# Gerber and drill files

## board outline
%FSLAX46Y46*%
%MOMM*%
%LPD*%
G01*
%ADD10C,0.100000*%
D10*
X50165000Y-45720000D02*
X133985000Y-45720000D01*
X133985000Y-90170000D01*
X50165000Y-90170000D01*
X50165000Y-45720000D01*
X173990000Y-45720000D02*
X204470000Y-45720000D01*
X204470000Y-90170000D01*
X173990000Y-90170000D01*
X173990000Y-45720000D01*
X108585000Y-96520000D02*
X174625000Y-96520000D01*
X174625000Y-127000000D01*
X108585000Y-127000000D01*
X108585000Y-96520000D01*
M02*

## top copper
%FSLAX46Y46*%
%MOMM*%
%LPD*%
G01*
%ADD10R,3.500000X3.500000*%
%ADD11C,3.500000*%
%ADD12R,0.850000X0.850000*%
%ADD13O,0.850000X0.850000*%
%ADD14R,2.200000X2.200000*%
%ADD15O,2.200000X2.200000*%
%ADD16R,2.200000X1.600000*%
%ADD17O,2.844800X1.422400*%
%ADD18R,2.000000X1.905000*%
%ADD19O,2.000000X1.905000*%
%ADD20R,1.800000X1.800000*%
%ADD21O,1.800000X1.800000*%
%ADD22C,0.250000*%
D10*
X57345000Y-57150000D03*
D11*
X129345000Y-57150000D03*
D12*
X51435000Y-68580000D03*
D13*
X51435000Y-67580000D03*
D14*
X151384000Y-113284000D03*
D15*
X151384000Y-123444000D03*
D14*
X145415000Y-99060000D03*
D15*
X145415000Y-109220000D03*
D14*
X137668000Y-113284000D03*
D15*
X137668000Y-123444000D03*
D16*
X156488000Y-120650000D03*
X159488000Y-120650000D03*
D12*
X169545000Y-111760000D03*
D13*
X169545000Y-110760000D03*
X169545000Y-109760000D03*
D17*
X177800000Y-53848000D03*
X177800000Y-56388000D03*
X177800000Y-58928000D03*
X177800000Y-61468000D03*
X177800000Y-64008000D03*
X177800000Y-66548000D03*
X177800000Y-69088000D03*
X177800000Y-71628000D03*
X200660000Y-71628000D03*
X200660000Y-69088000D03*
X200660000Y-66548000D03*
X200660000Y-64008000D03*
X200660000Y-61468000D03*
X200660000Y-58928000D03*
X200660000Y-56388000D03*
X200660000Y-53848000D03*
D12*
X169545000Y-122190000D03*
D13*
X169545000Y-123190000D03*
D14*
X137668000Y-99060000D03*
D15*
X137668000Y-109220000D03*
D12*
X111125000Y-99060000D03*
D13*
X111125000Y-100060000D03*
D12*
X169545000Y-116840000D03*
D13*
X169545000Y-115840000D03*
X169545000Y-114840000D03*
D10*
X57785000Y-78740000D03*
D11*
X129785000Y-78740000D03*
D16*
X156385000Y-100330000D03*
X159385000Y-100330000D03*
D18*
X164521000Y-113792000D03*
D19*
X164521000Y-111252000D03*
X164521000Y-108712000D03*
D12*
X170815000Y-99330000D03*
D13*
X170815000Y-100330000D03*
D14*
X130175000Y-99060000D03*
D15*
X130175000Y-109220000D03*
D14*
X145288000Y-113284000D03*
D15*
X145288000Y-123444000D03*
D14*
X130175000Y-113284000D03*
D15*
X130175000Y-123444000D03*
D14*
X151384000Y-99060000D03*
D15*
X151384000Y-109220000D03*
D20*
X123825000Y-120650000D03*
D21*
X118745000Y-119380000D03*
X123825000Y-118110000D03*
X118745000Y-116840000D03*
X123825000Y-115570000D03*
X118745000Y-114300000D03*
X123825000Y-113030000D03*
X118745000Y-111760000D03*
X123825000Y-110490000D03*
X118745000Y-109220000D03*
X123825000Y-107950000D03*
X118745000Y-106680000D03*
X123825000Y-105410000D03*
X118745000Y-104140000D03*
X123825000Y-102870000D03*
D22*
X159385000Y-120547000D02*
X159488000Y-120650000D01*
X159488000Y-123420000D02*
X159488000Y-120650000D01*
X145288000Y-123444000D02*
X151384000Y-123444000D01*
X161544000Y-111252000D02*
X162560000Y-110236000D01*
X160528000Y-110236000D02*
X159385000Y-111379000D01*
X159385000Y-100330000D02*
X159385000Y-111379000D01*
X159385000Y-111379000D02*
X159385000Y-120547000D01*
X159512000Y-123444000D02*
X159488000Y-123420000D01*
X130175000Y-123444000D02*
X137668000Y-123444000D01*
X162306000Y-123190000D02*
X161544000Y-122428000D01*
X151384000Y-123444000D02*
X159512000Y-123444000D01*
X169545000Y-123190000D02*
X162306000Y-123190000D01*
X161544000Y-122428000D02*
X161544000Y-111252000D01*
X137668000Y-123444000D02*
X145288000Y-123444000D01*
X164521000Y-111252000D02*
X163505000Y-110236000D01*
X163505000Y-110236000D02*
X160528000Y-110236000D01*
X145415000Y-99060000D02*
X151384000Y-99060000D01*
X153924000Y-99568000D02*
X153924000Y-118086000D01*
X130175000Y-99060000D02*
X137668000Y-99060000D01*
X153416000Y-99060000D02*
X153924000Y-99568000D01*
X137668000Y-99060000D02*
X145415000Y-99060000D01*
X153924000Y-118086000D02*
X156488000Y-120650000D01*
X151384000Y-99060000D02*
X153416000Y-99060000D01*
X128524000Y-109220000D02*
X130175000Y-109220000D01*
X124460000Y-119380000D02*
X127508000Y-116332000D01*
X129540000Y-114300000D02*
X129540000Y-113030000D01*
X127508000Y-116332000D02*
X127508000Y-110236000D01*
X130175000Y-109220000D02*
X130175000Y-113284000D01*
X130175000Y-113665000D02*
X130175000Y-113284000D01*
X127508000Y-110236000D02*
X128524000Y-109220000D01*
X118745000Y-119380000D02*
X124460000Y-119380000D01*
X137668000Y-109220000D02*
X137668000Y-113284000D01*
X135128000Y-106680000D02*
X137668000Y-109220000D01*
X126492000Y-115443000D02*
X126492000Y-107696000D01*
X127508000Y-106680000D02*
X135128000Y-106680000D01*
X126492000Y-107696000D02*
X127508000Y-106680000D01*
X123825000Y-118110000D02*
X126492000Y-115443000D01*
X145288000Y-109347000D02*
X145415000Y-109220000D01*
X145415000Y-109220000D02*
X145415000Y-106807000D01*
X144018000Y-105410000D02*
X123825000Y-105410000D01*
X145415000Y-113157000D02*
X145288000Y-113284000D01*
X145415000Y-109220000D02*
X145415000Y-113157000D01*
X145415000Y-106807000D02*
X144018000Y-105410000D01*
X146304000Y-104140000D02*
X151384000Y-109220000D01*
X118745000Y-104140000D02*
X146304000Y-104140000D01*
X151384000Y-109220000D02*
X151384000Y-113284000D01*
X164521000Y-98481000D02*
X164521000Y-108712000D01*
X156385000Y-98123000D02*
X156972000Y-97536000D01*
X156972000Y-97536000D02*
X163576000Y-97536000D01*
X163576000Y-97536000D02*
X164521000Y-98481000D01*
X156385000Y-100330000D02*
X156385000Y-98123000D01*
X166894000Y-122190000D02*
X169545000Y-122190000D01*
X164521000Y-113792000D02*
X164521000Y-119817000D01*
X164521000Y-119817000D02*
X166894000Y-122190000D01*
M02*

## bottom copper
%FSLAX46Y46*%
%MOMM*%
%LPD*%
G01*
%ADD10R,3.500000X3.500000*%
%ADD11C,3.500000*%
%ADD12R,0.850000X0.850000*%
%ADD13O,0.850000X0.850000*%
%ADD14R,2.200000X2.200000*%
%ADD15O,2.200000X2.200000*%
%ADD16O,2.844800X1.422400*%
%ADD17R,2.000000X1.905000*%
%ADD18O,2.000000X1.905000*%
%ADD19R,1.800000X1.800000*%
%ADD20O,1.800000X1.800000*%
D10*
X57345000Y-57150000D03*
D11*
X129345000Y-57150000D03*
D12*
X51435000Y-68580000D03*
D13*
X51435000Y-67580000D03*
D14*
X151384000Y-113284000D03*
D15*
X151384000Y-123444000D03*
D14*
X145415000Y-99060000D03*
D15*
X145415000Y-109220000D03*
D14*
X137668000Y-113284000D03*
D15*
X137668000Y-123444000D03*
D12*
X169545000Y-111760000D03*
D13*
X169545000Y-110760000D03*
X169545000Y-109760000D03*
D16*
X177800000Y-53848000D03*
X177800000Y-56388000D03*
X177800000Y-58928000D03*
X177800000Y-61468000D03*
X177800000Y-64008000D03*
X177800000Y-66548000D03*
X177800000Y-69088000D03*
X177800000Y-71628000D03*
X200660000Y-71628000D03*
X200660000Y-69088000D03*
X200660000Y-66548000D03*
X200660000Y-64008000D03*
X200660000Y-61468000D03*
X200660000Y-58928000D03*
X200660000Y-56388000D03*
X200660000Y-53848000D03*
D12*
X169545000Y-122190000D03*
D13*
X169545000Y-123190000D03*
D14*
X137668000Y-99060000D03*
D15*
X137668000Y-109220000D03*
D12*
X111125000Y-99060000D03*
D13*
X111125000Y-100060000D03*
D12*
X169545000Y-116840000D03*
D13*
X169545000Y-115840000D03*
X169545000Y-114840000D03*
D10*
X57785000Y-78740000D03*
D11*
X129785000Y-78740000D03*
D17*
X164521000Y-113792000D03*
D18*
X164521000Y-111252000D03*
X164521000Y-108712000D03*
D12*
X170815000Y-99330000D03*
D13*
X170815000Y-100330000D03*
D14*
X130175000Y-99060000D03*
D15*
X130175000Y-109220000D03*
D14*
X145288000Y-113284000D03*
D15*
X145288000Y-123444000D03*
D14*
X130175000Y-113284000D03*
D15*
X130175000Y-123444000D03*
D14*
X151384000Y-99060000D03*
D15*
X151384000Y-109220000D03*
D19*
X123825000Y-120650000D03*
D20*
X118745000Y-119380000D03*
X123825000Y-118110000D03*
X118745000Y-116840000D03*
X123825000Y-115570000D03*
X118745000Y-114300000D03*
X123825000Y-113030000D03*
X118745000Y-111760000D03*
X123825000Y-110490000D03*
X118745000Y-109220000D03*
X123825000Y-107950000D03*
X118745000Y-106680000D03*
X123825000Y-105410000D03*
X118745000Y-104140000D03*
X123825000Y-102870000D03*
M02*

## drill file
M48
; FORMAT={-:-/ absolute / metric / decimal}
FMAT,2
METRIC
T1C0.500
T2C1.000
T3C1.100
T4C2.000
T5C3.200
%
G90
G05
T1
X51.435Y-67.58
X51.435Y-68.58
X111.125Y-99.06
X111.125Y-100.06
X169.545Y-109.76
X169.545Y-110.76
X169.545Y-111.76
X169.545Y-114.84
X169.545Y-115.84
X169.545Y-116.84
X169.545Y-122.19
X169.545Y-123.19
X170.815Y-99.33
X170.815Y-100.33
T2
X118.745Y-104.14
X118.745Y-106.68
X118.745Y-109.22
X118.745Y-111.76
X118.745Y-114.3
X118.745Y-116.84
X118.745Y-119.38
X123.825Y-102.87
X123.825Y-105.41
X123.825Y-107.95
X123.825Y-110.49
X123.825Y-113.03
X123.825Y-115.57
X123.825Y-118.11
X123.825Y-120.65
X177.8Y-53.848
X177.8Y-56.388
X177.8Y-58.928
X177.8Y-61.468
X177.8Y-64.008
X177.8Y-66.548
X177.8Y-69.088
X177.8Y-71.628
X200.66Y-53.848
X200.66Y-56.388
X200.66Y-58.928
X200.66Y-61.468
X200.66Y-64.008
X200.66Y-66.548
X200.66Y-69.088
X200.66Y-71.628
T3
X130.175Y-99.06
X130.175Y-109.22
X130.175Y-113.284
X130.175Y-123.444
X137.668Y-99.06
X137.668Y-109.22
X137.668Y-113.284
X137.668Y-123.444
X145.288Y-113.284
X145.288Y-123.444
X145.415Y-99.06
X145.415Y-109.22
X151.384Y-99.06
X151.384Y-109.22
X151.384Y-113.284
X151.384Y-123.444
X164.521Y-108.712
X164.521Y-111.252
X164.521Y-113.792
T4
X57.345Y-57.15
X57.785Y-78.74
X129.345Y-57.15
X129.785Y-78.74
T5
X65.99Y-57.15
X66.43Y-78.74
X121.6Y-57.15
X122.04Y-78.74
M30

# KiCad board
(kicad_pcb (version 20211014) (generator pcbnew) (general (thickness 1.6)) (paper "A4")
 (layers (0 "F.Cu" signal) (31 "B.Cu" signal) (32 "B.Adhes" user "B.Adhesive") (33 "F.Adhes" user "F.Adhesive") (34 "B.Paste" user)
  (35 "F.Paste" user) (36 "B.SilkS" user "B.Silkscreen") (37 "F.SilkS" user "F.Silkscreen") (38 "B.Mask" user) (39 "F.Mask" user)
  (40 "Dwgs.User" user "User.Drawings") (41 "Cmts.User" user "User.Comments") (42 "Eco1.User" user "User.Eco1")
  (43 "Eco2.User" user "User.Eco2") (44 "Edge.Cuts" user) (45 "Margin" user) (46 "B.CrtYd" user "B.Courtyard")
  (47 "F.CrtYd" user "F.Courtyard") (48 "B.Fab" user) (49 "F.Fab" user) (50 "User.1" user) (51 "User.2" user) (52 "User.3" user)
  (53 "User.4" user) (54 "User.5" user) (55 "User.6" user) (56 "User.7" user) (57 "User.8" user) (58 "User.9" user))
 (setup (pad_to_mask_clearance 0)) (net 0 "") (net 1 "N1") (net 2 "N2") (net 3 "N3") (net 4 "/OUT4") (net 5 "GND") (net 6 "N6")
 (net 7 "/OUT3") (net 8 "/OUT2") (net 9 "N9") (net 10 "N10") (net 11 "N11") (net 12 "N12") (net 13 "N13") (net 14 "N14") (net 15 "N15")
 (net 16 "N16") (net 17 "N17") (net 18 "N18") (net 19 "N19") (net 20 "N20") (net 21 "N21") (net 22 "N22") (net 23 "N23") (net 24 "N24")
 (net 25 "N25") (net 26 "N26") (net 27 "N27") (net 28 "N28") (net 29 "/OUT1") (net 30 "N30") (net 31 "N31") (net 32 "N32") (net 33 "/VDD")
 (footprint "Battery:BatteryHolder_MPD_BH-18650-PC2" (layer "F.Cu") (at 57.345 57.15)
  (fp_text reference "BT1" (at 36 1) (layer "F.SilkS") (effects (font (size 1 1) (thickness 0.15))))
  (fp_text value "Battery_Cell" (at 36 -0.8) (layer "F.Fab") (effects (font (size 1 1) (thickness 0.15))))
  (pad "" np_thru_hole circle (at 8.645 0) (size 3.2 3.2) (drill 3.2) (layers *.Cu *.Mask))
  (pad "" np_thru_hole circle (at 64.255 0) (size 3.2 3.2) (drill 3.2) (layers *.Cu *.Mask))
  (pad "1" thru_hole rect (at 0 0) (size 3.5 3.5) (drill 2) (layers *.Cu *.Mask) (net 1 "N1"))
  (pad "2" thru_hole circle (at 72 0) (size 3.5 3.5) (drill 2) (layers *.Cu *.Mask) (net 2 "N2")))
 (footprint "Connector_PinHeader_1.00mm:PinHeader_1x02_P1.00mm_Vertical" (layer "F.Cu") (at 51.435 68.58 180)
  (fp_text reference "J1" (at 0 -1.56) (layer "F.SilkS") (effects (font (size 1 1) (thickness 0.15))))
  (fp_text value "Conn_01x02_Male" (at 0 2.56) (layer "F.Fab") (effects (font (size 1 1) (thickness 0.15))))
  (pad "1" thru_hole rect (at 0 0 180) (size 0.85 0.85) (drill 0.5) (layers *.Cu *.Mask) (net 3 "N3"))
  (pad "2" thru_hole oval (at 0 1 180) (size 0.85 0.85) (drill 0.5) (layers *.Cu *.Mask) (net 1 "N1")))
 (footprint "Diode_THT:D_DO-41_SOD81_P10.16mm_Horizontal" (layer "F.Cu") (at 151.384 113.284 -90)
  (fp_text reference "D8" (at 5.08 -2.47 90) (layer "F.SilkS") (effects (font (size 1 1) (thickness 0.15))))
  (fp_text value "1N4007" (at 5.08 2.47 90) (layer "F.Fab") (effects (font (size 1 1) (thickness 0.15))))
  (pad "1" thru_hole rect (at 0 0 270) (size 2.2 2.2) (drill 1.1) (layers *.Cu *.Mask) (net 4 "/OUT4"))
  (pad "2" thru_hole oval (at 10.16 0 270) (size 2.2 2.2) (drill 1.1) (layers *.Cu *.Mask) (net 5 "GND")))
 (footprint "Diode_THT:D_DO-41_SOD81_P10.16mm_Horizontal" (layer "F.Cu") (at 145.415 99.06 -90)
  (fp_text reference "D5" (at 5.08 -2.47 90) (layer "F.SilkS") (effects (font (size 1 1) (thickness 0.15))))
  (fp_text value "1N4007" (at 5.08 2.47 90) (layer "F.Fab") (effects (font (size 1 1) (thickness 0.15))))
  (pad "1" thru_hole rect (at 0 0 270) (size 2.2 2.2) (drill 1.1) (layers *.Cu *.Mask) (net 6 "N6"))
  (pad "2" thru_hole oval (at 10.16 0 270) (size 2.2 2.2) (drill 1.1) (layers *.Cu *.Mask) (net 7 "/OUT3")))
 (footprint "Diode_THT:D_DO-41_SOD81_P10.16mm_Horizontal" (layer "F.Cu") (at 137.668 113.284 -90)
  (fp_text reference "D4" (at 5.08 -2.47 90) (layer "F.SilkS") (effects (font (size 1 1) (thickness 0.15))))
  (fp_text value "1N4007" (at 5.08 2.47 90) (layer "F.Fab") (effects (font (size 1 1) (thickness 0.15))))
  (pad "1" thru_hole rect (at 0 0 270) (size 2.2 2.2) (drill 1.1) (layers *.Cu *.Mask) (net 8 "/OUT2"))
  (pad "2" thru_hole oval (at 10.16 0 270) (size 2.2 2.2) (drill 1.1) (layers *.Cu *.Mask) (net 5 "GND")))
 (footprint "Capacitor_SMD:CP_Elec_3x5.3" (layer "F.Cu") (at 157.988 120.65)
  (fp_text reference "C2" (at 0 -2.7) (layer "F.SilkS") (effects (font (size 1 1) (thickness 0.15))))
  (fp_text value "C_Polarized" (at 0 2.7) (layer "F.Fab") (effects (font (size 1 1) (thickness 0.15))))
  (pad "1" smd rect (at -1.5 0) (size 2.2 1.6) (layers "F.Cu" "F.Paste" "F.Mask") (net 6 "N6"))
  (pad "2" smd rect (at 1.5 0) (size 2.2 1.6) (layers "F.Cu" "F.Paste" "F.Mask") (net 5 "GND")))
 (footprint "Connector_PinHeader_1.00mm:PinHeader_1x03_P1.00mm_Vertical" (layer "F.Cu") (at 169.545 111.76 180)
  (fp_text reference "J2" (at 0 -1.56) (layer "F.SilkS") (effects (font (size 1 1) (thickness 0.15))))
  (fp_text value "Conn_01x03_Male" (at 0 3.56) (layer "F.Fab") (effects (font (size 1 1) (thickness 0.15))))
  (pad "1" thru_hole rect (at 0 0 180) (size 0.85 0.85) (drill 0.5) (layers *.Cu *.Mask) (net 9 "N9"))
  (pad "2" thru_hole oval (at 0 1 180) (size 0.85 0.85) (drill 0.5) (layers *.Cu *.Mask) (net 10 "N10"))
  (pad "3" thru_hole oval (at 0 2 180) (size 0.85 0.85) (drill 0.5) (layers *.Cu *.Mask) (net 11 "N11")))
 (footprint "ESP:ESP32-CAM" (layer "F.Cu") (at 189.23 64.008)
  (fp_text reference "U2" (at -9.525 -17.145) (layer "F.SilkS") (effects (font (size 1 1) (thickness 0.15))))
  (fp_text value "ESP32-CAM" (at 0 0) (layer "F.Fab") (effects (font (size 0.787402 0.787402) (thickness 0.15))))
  (pad "1" thru_hole oval (at -11.43 -10.16) (size 2.8448 1.4224) (drill 1) (layers *.Cu *.Mask) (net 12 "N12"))
  (pad "2" thru_hole oval (at -11.43 -7.62) (size 2.8448 1.4224) (drill 1) (layers *.Cu *.Mask) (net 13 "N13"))
  (pad "3" thru_hole oval (at -11.43 -5.08) (size 2.8448 1.4224) (drill 1) (layers *.Cu *.Mask) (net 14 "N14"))
  (pad "4" thru_hole oval (at -11.43 -2.54) (size 2.8448 1.4224) (drill 1) (layers *.Cu *.Mask) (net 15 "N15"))
  (pad "5" thru_hole oval (at -11.43 0) (size 2.8448 1.4224) (drill 1) (layers *.Cu *.Mask) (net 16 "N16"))
  (pad "6" thru_hole oval (at -11.43 2.54) (size 2.8448 1.4224) (drill 1) (layers *.Cu *.Mask) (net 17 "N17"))
  (pad "7" thru_hole oval (at -11.43 5.08) (size 2.8448 1.4224) (drill 1) (layers *.Cu *.Mask) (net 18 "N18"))
  (pad "8" thru_hole oval (at -11.43 7.62) (size 2.8448 1.4224) (drill 1) (layers *.Cu *.Mask) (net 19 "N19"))
  (pad "9" thru_hole oval (at 11.43 7.62) (size 2.8448 1.4224) (drill 1) (layers *.Cu *.Mask) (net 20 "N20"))
  (pad "10" thru_hole oval (at 11.43 5.08) (size 2.8448 1.4224) (drill 1) (layers *.Cu *.Mask) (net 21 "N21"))
  (pad "11" thru_hole oval (at 11.43 2.54) (size 2.8448 1.4224) (drill 1) (layers *.Cu *.Mask) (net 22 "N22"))
  (pad "12" thru_hole oval (at 11.43 0) (size 2.8448 1.4224) (drill 1) (layers *.Cu *.Mask) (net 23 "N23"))
  (pad "13" thru_hole oval (at 11.43 -2.54) (size 2.8448 1.4224) (drill 1) (layers *.Cu *.Mask) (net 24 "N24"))
  (pad "14" thru_hole oval (at 11.43 -5.08) (size 2.8448 1.4224) (drill 1) (layers *.Cu *.Mask) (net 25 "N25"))
  (pad "15" thru_hole oval (at 11.43 -7.62) (size 2.8448 1.4224) (drill 1) (layers *.Cu *.Mask) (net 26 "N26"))
  (pad "16" thru_hole oval (at 11.43 -10.16) (size 2.8448 1.4224) (drill 1) (layers *.Cu *.Mask) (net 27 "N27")))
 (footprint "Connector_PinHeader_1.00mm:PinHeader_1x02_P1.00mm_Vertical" (layer "F.Cu") (at 169.545 122.19)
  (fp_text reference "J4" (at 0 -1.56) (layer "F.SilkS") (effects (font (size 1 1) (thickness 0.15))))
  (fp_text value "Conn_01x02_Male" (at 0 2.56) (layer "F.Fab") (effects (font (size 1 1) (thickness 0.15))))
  (pad "1" thru_hole rect (at 0 0) (size 0.85 0.85) (drill 0.5) (layers *.Cu *.Mask) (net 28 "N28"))
  (pad "2" thru_hole oval (at 0 1) (size 0.85 0.85) (drill 0.5) (layers *.Cu *.Mask) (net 5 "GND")))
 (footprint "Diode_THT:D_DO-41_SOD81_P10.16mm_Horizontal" (layer "F.Cu") (at 137.668 99.06 -90)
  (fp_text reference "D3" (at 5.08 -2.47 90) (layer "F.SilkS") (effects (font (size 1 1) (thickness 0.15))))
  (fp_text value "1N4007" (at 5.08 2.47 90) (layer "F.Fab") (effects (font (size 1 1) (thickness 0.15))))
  (pad "1" thru_hole rect (at 0 0 270) (size 2.2 2.2) (drill 1.1) (layers *.Cu *.Mask) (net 6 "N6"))
  (pad "2" thru_hole oval (at 10.16 0 270) (size 2.2 2.2) (drill 1.1) (layers *.Cu *.Mask) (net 8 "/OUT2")))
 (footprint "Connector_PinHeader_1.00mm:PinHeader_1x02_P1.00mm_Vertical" (layer "F.Cu") (at 111.125 99.06)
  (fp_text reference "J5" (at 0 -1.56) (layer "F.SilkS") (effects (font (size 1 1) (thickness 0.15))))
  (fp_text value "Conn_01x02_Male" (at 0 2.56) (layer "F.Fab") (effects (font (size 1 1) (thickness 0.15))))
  (pad "1" thru_hole rect (at 0 0) (size 0.85 0.85) (drill 0.5) (layers *.Cu *.Mask) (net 8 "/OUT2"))
  (pad "2" thru_hole oval (at 0 1) (size 0.85 0.85) (drill 0.5) (layers *.Cu *.Mask) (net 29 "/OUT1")))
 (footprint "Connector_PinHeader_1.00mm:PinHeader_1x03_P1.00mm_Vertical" (layer "F.Cu") (at 169.545 116.84 180)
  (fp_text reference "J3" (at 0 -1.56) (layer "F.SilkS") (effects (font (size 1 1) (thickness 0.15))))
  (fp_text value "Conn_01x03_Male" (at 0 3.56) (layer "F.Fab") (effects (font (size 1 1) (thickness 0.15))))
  (pad "1" thru_hole rect (at 0 0 180) (size 0.85 0.85) (drill 0.5) (layers *.Cu *.Mask) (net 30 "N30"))
  (pad "2" thru_hole oval (at 0 1 180) (size 0.85 0.85) (drill 0.5) (layers *.Cu *.Mask) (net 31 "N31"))
  (pad "3" thru_hole oval (at 0 2 180) (size 0.85 0.85) (drill 0.5) (layers *.Cu *.Mask) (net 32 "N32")))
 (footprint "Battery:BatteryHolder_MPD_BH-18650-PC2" (layer "F.Cu") (at 57.785 78.74)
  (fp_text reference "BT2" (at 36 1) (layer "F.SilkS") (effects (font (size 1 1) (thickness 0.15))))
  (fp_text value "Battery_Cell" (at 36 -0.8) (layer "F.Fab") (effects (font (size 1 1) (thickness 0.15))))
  (pad "" np_thru_hole circle (at 64.255 0) (size 3.2 3.2) (drill 3.2) (layers *.Cu *.Mask))
  (pad "" np_thru_hole circle (at 8.645 0) (size 3.2 3.2) (drill 3.2) (layers *.Cu *.Mask))
  (pad "1" thru_hole rect (at 0 0) (size 3.5 3.5) (drill 2) (layers *.Cu *.Mask) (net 2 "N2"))
  (pad "2" thru_hole circle (at 72 0) (size 3.5 3.5) (drill 2) (layers *.Cu *.Mask) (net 3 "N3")))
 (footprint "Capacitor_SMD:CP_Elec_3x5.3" (layer "F.Cu") (at 157.885 100.33)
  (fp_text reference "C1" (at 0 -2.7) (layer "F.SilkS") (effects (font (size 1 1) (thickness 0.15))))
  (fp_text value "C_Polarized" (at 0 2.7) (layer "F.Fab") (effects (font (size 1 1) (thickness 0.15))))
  (pad "1" smd rect (at -1.5 0) (size 2.2 1.6) (layers "F.Cu" "F.Paste" "F.Mask") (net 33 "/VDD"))
  (pad "2" smd rect (at 1.5 0) (size 2.2 1.6) (layers "F.Cu" "F.Paste" "F.Mask") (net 5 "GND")))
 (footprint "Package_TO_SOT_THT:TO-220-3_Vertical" (layer "F.Cu") (at 164.521 113.792 90)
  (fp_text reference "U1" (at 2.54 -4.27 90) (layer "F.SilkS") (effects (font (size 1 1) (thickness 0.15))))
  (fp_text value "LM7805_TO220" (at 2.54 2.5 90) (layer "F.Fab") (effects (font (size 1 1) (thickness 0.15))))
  (pad "1" thru_hole rect (at 0 0 90) (size 1.905 2) (drill 1.1) (layers *.Cu *.Mask) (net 28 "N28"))
  (pad "2" thru_hole oval (at 2.54 0 90) (size 1.905 2) (drill 1.1) (layers *.Cu *.Mask) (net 5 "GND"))
  (pad "3" thru_hole oval (at 5.08 0 90) (size 1.905 2) (drill 1.1) (layers *.Cu *.Mask) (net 33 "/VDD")))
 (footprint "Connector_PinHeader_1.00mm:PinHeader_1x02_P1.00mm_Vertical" (layer "F.Cu") (at 170.815 99.33)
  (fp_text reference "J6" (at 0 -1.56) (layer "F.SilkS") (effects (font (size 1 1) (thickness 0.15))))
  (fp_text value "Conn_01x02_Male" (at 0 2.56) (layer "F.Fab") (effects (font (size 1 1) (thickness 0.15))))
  (pad "1" thru_hole rect (at 0 0) (size 0.85 0.85) (drill 0.5) (layers *.Cu *.Mask) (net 4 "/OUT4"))
  (pad "2" thru_hole oval (at 0 1) (size 0.85 0.85) (drill 0.5) (layers *.Cu *.Mask) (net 7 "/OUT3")))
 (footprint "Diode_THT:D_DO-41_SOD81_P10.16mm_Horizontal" (layer "F.Cu") (at 130.175 99.06 -90)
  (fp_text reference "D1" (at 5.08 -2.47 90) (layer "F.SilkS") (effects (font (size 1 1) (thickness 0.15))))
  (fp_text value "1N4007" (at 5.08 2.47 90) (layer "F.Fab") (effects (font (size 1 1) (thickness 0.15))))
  (pad "1" thru_hole rect (at 0 0 270) (size 2.2 2.2) (drill 1.1) (layers *.Cu *.Mask) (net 6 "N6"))
  (pad "2" thru_hole oval (at 10.16 0 270) (size 2.2 2.2) (drill 1.1) (layers *.Cu *.Mask) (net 29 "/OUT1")))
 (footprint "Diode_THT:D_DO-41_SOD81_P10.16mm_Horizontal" (layer "F.Cu") (at 145.288 113.284 -90)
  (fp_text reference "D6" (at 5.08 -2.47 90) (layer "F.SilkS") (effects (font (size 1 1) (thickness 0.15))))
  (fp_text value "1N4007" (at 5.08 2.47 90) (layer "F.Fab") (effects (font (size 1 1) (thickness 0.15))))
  (pad "1" thru_hole rect (at 0 0 270) (size 2.2 2.2) (drill 1.1) (layers *.Cu *.Mask) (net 7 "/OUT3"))
  (pad "2" thru_hole oval (at 10.16 0 270) (size 2.2 2.2) (drill 1.1) (layers *.Cu *.Mask) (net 5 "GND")))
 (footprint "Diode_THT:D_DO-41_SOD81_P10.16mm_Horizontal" (layer "F.Cu") (at 130.175 113.284 -90)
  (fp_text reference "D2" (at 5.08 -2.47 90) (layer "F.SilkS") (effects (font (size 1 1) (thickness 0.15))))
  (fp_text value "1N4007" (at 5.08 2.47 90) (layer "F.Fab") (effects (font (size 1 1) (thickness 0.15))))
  (pad "1" thru_hole rect (at 0 0 270) (size 2.2 2.2) (drill 1.1) (layers *.Cu *.Mask) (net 29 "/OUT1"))
  (pad "2" thru_hole oval (at 10.16 0 270) (size 2.2 2.2) (drill 1.1) (layers *.Cu *.Mask) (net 5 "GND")))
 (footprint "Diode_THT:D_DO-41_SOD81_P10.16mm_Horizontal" (layer "F.Cu") (at 151.384 99.06 -90)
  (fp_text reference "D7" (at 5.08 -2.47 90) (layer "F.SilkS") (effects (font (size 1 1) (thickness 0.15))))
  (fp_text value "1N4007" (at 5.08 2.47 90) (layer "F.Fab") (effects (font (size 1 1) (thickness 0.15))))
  (pad "1" thru_hole rect (at 0 0 270) (size 2.2 2.2) (drill 1.1) (layers *.Cu *.Mask) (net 6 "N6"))
  (pad "2" thru_hole oval (at 10.16 0 270) (size 2.2 2.2) (drill 1.1) (layers *.Cu *.Mask) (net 4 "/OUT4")))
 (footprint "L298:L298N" (layer "F.Cu") (at 120.7686 111.8648 90)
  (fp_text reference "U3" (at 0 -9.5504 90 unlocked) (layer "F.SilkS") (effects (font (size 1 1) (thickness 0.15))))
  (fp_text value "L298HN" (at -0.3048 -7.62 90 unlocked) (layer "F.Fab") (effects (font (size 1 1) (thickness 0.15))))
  (pad "1" thru_hole rect (at -8.7852 3.0564 90) (size 1.8 1.8) (drill 1) (layers *.Cu *.Mask) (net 5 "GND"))
  (pad "2" thru_hole oval (at -7.5152 -2.0236 90) (size 1.8 1.8) (drill 1) (layers *.Cu *.Mask) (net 29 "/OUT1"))
  (pad "3" thru_hole oval (at -6.2452 3.0564 90) (size 1.8 1.8) (drill 1) (layers *.Cu *.Mask) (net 8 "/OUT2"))
  (pad "4" thru_hole oval (at -4.9752 -2.0236 90) (size 1.8 1.8) (drill 1) (layers *.Cu *.Mask) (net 6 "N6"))
  (pad "5" thru_hole oval (at -3.7052 3.0564 90) (size 1.8 1.8) (drill 1) (layers *.Cu *.Mask) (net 9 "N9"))
  (pad "6" thru_hole oval (at -2.4352 -2.0236 90) (size 1.8 1.8) (drill 1) (layers *.Cu *.Mask) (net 11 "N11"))
  (pad "7" thru_hole oval (at -1.1652 3.0564 90) (size 1.8 1.8) (drill 1) (layers *.Cu *.Mask) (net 10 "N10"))
  (pad "8" thru_hole oval (at 0.1048 -2.0236 90) (size 1.8 1.8) (drill 1) (layers *.Cu *.Mask) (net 5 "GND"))
  (pad "9" thru_hole oval (at 1.3748 3.0564 90) (size 1.8 1.8) (drill 1) (layers *.Cu *.Mask) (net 33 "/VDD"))
  (pad "10" thru_hole oval (at 2.6448 -2.0236 90) (size 1.8 1.8) (drill 1) (layers *.Cu *.Mask) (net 30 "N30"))
  (pad "11" thru_hole oval (at 3.9148 3.0564 90) (size 1.8 1.8) (drill 1) (layers *.Cu *.Mask) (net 32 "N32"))
  (pad "12" thru_hole oval (at 5.1848 -2.0236 90) (size 1.8 1.8) (drill 1) (layers *.Cu *.Mask) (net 31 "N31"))
  (pad "13" thru_hole oval (at 6.4548 3.0564 90) (size 1.8 1.8) (drill 1) (layers *.Cu *.Mask) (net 7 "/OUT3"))
  (pad "14" thru_hole oval (at 7.7248 -2.0236 90) (size 1.8 1.8) (drill 1) (layers *.Cu *.Mask) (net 4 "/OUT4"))
  (pad "15" thru_hole oval (at 8.9948 3.0564 90) (size 1.8 1.8) (drill 1) (layers *.Cu *.Mask) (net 5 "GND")))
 (gr_rect (start 50.165 45.72) (end 133.985 90.17) (layer "Edge.Cuts") (width 0.1) (fill none))
 (gr_rect (start 173.99 45.72) (end 204.47 90.17) (layer "Edge.Cuts") (width 0.1) (fill none))
 (gr_rect (start 108.585 96.52) (end 174.625 127) (layer "Edge.Cuts") (width 0.1) (fill none))
 (segment (start 159.385 120.547) (end 159.488 120.65) (width 0.25) (layer "F.Cu") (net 5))
 (segment (start 159.488 123.42) (end 159.488 120.65) (width 0.25) (layer "F.Cu") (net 5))
 (segment (start 145.288 123.444) (end 151.384 123.444) (width 0.25) (layer "F.Cu") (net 5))
 (segment (start 161.544 111.252) (end 162.56 110.236) (width 0.25) (layer "F.Cu") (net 5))
 (segment (start 160.528 110.236) (end 159.385 111.379) (width 0.25) (layer "F.Cu") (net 5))
 (segment (start 159.385 100.33) (end 159.385 111.379) (width 0.25) (layer "F.Cu") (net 5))
 (segment (start 159.385 111.379) (end 159.385 120.547) (width 0.25) (layer "F.Cu") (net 5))
 (segment (start 159.512 123.444) (end 159.488 123.42) (width 0.25) (layer "F.Cu") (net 5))
 (segment (start 130.175 123.444) (end 137.668 123.444) (width 0.25) (layer "F.Cu") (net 5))
 (segment (start 162.306 123.19) (end 161.544 122.428) (width 0.25) (layer "F.Cu") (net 5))
 (segment (start 151.384 123.444) (end 159.512 123.444) (width 0.25) (layer "F.Cu") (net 5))
 (segment (start 169.545 123.19) (end 162.306 123.19) (width 0.25) (layer "F.Cu") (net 5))
 (segment (start 161.544 122.428) (end 161.544 111.252) (width 0.25) (layer "F.Cu") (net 5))
 (segment (start 137.668 123.444) (end 145.288 123.444) (width 0.25) (layer "F.Cu") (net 5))
 (segment (start 164.521 111.252) (end 163.505 110.236) (width 0.25) (layer "F.Cu") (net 5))
 (segment (start 163.505 110.236) (end 160.528 110.236) (width 0.25) (layer "F.Cu") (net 5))
 (segment (start 145.415 99.06) (end 151.384 99.06) (width 0.25) (layer "F.Cu") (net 6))
 (segment (start 153.924 99.568) (end 153.924 118.086) (width 0.25) (layer "F.Cu") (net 6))
 (segment (start 130.175 99.06) (end 137.668 99.06) (width 0.25) (layer "F.Cu") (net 6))
 (segment (start 153.416 99.06) (end 153.924 99.568) (width 0.25) (layer "F.Cu") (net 6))
 (segment (start 137.668 99.06) (end 145.415 99.06) (width 0.25) (layer "F.Cu") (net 6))
 (segment (start 153.924 118.086) (end 156.488 120.65) (width 0.25) (layer "F.Cu") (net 6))
 (segment (start 151.384 99.06) (end 153.416 99.06) (width 0.25) (layer "F.Cu") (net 6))
 (segment (start 128.524 109.22) (end 130.175 109.22) (width 0.25) (layer "F.Cu") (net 29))
 (segment (start 124.46 119.38) (end 127.508 116.332) (width 0.25) (layer "F.Cu") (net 29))
 (segment (start 129.54 114.3) (end 129.54 113.03) (width 0.25) (layer "F.Cu") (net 29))
 (segment (start 127.508 116.332) (end 127.508 110.236) (width 0.25) (layer "F.Cu") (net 29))
 (segment (start 130.175 109.22) (end 130.175 113.284) (width 0.25) (layer "F.Cu") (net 29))
 (segment (start 130.175 113.665) (end 130.175 113.284) (width 0.25) (layer "F.Cu") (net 29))
 (segment (start 127.508 110.236) (end 128.524 109.22) (width 0.25) (layer "F.Cu") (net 29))
 (segment (start 118.745 119.38) (end 124.46 119.38) (width 0.25) (layer "F.Cu") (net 29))
 (segment (start 137.668 109.22) (end 137.668 113.284) (width 0.25) (layer "F.Cu") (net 8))
 (segment (start 135.128 106.68) (end 137.668 109.22) (width 0.25) (layer "F.Cu") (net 8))
 (segment (start 126.492 115.443) (end 126.492 107.696) (width 0.25) (layer "F.Cu") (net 8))
 (segment (start 127.508 106.68) (end 135.128 106.68) (width 0.25) (layer "F.Cu") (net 8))
 (segment (start 126.492 107.696) (end 127.508 106.68) (width 0.25) (layer "F.Cu") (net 8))
 (segment (start 123.825 118.11) (end 126.492 115.443) (width 0.25) (layer "F.Cu") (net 8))
 (segment (start 145.288 109.347) (end 145.415 109.22) (width 0.25) (layer "F.Cu") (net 7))
 (segment (start 145.415 109.22) (end 145.415 106.807) (width 0.25) (layer "F.Cu") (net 7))
 (segment (start 144.018 105.41) (end 123.825 105.41) (width 0.25) (layer "F.Cu") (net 7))
 (segment (start 145.415 113.157) (end 145.288 113.284) (width 0.25) (layer "F.Cu") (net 7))
 (segment (start 145.415 109.22) (end 145.415 113.157) (width 0.25) (layer "F.Cu") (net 7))
 (segment (start 145.415 106.807) (end 144.018 105.41) (width 0.25) (layer "F.Cu") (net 7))
 (segment (start 146.304 104.14) (end 151.384 109.22) (width 0.25) (layer "F.Cu") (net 4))
 (segment (start 118.745 104.14) (end 146.304 104.14) (width 0.25) (layer "F.Cu") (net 4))
 (segment (start 151.384 109.22) (end 151.384 113.284) (width 0.25) (layer "F.Cu") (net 4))
 (segment (start 164.521 98.481) (end 164.521 108.712) (width 0.25) (layer "F.Cu") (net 33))
 (segment (start 156.385 98.123) (end 156.972 97.536) (width 0.25) (layer "F.Cu") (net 33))
 (segment (start 156.972 97.536) (end 163.576 97.536) (width 0.25) (layer "F.Cu") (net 33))
 (segment (start 163.576 97.536) (end 164.521 98.481) (width 0.25) (layer "F.Cu") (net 33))
 (segment (start 156.385 100.33) (end 156.385 98.123) (width 0.25) (layer "F.Cu") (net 33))
 (segment (start 166.894 122.19) (end 169.545 122.19) (width 0.25) (layer "F.Cu") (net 28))
 (segment (start 164.521 113.792) (end 164.521 119.817) (width 0.25) (layer "F.Cu") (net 28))
 (segment (start 164.521 119.817) (end 166.894 122.19) (width 0.25) (layer "F.Cu") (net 28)))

